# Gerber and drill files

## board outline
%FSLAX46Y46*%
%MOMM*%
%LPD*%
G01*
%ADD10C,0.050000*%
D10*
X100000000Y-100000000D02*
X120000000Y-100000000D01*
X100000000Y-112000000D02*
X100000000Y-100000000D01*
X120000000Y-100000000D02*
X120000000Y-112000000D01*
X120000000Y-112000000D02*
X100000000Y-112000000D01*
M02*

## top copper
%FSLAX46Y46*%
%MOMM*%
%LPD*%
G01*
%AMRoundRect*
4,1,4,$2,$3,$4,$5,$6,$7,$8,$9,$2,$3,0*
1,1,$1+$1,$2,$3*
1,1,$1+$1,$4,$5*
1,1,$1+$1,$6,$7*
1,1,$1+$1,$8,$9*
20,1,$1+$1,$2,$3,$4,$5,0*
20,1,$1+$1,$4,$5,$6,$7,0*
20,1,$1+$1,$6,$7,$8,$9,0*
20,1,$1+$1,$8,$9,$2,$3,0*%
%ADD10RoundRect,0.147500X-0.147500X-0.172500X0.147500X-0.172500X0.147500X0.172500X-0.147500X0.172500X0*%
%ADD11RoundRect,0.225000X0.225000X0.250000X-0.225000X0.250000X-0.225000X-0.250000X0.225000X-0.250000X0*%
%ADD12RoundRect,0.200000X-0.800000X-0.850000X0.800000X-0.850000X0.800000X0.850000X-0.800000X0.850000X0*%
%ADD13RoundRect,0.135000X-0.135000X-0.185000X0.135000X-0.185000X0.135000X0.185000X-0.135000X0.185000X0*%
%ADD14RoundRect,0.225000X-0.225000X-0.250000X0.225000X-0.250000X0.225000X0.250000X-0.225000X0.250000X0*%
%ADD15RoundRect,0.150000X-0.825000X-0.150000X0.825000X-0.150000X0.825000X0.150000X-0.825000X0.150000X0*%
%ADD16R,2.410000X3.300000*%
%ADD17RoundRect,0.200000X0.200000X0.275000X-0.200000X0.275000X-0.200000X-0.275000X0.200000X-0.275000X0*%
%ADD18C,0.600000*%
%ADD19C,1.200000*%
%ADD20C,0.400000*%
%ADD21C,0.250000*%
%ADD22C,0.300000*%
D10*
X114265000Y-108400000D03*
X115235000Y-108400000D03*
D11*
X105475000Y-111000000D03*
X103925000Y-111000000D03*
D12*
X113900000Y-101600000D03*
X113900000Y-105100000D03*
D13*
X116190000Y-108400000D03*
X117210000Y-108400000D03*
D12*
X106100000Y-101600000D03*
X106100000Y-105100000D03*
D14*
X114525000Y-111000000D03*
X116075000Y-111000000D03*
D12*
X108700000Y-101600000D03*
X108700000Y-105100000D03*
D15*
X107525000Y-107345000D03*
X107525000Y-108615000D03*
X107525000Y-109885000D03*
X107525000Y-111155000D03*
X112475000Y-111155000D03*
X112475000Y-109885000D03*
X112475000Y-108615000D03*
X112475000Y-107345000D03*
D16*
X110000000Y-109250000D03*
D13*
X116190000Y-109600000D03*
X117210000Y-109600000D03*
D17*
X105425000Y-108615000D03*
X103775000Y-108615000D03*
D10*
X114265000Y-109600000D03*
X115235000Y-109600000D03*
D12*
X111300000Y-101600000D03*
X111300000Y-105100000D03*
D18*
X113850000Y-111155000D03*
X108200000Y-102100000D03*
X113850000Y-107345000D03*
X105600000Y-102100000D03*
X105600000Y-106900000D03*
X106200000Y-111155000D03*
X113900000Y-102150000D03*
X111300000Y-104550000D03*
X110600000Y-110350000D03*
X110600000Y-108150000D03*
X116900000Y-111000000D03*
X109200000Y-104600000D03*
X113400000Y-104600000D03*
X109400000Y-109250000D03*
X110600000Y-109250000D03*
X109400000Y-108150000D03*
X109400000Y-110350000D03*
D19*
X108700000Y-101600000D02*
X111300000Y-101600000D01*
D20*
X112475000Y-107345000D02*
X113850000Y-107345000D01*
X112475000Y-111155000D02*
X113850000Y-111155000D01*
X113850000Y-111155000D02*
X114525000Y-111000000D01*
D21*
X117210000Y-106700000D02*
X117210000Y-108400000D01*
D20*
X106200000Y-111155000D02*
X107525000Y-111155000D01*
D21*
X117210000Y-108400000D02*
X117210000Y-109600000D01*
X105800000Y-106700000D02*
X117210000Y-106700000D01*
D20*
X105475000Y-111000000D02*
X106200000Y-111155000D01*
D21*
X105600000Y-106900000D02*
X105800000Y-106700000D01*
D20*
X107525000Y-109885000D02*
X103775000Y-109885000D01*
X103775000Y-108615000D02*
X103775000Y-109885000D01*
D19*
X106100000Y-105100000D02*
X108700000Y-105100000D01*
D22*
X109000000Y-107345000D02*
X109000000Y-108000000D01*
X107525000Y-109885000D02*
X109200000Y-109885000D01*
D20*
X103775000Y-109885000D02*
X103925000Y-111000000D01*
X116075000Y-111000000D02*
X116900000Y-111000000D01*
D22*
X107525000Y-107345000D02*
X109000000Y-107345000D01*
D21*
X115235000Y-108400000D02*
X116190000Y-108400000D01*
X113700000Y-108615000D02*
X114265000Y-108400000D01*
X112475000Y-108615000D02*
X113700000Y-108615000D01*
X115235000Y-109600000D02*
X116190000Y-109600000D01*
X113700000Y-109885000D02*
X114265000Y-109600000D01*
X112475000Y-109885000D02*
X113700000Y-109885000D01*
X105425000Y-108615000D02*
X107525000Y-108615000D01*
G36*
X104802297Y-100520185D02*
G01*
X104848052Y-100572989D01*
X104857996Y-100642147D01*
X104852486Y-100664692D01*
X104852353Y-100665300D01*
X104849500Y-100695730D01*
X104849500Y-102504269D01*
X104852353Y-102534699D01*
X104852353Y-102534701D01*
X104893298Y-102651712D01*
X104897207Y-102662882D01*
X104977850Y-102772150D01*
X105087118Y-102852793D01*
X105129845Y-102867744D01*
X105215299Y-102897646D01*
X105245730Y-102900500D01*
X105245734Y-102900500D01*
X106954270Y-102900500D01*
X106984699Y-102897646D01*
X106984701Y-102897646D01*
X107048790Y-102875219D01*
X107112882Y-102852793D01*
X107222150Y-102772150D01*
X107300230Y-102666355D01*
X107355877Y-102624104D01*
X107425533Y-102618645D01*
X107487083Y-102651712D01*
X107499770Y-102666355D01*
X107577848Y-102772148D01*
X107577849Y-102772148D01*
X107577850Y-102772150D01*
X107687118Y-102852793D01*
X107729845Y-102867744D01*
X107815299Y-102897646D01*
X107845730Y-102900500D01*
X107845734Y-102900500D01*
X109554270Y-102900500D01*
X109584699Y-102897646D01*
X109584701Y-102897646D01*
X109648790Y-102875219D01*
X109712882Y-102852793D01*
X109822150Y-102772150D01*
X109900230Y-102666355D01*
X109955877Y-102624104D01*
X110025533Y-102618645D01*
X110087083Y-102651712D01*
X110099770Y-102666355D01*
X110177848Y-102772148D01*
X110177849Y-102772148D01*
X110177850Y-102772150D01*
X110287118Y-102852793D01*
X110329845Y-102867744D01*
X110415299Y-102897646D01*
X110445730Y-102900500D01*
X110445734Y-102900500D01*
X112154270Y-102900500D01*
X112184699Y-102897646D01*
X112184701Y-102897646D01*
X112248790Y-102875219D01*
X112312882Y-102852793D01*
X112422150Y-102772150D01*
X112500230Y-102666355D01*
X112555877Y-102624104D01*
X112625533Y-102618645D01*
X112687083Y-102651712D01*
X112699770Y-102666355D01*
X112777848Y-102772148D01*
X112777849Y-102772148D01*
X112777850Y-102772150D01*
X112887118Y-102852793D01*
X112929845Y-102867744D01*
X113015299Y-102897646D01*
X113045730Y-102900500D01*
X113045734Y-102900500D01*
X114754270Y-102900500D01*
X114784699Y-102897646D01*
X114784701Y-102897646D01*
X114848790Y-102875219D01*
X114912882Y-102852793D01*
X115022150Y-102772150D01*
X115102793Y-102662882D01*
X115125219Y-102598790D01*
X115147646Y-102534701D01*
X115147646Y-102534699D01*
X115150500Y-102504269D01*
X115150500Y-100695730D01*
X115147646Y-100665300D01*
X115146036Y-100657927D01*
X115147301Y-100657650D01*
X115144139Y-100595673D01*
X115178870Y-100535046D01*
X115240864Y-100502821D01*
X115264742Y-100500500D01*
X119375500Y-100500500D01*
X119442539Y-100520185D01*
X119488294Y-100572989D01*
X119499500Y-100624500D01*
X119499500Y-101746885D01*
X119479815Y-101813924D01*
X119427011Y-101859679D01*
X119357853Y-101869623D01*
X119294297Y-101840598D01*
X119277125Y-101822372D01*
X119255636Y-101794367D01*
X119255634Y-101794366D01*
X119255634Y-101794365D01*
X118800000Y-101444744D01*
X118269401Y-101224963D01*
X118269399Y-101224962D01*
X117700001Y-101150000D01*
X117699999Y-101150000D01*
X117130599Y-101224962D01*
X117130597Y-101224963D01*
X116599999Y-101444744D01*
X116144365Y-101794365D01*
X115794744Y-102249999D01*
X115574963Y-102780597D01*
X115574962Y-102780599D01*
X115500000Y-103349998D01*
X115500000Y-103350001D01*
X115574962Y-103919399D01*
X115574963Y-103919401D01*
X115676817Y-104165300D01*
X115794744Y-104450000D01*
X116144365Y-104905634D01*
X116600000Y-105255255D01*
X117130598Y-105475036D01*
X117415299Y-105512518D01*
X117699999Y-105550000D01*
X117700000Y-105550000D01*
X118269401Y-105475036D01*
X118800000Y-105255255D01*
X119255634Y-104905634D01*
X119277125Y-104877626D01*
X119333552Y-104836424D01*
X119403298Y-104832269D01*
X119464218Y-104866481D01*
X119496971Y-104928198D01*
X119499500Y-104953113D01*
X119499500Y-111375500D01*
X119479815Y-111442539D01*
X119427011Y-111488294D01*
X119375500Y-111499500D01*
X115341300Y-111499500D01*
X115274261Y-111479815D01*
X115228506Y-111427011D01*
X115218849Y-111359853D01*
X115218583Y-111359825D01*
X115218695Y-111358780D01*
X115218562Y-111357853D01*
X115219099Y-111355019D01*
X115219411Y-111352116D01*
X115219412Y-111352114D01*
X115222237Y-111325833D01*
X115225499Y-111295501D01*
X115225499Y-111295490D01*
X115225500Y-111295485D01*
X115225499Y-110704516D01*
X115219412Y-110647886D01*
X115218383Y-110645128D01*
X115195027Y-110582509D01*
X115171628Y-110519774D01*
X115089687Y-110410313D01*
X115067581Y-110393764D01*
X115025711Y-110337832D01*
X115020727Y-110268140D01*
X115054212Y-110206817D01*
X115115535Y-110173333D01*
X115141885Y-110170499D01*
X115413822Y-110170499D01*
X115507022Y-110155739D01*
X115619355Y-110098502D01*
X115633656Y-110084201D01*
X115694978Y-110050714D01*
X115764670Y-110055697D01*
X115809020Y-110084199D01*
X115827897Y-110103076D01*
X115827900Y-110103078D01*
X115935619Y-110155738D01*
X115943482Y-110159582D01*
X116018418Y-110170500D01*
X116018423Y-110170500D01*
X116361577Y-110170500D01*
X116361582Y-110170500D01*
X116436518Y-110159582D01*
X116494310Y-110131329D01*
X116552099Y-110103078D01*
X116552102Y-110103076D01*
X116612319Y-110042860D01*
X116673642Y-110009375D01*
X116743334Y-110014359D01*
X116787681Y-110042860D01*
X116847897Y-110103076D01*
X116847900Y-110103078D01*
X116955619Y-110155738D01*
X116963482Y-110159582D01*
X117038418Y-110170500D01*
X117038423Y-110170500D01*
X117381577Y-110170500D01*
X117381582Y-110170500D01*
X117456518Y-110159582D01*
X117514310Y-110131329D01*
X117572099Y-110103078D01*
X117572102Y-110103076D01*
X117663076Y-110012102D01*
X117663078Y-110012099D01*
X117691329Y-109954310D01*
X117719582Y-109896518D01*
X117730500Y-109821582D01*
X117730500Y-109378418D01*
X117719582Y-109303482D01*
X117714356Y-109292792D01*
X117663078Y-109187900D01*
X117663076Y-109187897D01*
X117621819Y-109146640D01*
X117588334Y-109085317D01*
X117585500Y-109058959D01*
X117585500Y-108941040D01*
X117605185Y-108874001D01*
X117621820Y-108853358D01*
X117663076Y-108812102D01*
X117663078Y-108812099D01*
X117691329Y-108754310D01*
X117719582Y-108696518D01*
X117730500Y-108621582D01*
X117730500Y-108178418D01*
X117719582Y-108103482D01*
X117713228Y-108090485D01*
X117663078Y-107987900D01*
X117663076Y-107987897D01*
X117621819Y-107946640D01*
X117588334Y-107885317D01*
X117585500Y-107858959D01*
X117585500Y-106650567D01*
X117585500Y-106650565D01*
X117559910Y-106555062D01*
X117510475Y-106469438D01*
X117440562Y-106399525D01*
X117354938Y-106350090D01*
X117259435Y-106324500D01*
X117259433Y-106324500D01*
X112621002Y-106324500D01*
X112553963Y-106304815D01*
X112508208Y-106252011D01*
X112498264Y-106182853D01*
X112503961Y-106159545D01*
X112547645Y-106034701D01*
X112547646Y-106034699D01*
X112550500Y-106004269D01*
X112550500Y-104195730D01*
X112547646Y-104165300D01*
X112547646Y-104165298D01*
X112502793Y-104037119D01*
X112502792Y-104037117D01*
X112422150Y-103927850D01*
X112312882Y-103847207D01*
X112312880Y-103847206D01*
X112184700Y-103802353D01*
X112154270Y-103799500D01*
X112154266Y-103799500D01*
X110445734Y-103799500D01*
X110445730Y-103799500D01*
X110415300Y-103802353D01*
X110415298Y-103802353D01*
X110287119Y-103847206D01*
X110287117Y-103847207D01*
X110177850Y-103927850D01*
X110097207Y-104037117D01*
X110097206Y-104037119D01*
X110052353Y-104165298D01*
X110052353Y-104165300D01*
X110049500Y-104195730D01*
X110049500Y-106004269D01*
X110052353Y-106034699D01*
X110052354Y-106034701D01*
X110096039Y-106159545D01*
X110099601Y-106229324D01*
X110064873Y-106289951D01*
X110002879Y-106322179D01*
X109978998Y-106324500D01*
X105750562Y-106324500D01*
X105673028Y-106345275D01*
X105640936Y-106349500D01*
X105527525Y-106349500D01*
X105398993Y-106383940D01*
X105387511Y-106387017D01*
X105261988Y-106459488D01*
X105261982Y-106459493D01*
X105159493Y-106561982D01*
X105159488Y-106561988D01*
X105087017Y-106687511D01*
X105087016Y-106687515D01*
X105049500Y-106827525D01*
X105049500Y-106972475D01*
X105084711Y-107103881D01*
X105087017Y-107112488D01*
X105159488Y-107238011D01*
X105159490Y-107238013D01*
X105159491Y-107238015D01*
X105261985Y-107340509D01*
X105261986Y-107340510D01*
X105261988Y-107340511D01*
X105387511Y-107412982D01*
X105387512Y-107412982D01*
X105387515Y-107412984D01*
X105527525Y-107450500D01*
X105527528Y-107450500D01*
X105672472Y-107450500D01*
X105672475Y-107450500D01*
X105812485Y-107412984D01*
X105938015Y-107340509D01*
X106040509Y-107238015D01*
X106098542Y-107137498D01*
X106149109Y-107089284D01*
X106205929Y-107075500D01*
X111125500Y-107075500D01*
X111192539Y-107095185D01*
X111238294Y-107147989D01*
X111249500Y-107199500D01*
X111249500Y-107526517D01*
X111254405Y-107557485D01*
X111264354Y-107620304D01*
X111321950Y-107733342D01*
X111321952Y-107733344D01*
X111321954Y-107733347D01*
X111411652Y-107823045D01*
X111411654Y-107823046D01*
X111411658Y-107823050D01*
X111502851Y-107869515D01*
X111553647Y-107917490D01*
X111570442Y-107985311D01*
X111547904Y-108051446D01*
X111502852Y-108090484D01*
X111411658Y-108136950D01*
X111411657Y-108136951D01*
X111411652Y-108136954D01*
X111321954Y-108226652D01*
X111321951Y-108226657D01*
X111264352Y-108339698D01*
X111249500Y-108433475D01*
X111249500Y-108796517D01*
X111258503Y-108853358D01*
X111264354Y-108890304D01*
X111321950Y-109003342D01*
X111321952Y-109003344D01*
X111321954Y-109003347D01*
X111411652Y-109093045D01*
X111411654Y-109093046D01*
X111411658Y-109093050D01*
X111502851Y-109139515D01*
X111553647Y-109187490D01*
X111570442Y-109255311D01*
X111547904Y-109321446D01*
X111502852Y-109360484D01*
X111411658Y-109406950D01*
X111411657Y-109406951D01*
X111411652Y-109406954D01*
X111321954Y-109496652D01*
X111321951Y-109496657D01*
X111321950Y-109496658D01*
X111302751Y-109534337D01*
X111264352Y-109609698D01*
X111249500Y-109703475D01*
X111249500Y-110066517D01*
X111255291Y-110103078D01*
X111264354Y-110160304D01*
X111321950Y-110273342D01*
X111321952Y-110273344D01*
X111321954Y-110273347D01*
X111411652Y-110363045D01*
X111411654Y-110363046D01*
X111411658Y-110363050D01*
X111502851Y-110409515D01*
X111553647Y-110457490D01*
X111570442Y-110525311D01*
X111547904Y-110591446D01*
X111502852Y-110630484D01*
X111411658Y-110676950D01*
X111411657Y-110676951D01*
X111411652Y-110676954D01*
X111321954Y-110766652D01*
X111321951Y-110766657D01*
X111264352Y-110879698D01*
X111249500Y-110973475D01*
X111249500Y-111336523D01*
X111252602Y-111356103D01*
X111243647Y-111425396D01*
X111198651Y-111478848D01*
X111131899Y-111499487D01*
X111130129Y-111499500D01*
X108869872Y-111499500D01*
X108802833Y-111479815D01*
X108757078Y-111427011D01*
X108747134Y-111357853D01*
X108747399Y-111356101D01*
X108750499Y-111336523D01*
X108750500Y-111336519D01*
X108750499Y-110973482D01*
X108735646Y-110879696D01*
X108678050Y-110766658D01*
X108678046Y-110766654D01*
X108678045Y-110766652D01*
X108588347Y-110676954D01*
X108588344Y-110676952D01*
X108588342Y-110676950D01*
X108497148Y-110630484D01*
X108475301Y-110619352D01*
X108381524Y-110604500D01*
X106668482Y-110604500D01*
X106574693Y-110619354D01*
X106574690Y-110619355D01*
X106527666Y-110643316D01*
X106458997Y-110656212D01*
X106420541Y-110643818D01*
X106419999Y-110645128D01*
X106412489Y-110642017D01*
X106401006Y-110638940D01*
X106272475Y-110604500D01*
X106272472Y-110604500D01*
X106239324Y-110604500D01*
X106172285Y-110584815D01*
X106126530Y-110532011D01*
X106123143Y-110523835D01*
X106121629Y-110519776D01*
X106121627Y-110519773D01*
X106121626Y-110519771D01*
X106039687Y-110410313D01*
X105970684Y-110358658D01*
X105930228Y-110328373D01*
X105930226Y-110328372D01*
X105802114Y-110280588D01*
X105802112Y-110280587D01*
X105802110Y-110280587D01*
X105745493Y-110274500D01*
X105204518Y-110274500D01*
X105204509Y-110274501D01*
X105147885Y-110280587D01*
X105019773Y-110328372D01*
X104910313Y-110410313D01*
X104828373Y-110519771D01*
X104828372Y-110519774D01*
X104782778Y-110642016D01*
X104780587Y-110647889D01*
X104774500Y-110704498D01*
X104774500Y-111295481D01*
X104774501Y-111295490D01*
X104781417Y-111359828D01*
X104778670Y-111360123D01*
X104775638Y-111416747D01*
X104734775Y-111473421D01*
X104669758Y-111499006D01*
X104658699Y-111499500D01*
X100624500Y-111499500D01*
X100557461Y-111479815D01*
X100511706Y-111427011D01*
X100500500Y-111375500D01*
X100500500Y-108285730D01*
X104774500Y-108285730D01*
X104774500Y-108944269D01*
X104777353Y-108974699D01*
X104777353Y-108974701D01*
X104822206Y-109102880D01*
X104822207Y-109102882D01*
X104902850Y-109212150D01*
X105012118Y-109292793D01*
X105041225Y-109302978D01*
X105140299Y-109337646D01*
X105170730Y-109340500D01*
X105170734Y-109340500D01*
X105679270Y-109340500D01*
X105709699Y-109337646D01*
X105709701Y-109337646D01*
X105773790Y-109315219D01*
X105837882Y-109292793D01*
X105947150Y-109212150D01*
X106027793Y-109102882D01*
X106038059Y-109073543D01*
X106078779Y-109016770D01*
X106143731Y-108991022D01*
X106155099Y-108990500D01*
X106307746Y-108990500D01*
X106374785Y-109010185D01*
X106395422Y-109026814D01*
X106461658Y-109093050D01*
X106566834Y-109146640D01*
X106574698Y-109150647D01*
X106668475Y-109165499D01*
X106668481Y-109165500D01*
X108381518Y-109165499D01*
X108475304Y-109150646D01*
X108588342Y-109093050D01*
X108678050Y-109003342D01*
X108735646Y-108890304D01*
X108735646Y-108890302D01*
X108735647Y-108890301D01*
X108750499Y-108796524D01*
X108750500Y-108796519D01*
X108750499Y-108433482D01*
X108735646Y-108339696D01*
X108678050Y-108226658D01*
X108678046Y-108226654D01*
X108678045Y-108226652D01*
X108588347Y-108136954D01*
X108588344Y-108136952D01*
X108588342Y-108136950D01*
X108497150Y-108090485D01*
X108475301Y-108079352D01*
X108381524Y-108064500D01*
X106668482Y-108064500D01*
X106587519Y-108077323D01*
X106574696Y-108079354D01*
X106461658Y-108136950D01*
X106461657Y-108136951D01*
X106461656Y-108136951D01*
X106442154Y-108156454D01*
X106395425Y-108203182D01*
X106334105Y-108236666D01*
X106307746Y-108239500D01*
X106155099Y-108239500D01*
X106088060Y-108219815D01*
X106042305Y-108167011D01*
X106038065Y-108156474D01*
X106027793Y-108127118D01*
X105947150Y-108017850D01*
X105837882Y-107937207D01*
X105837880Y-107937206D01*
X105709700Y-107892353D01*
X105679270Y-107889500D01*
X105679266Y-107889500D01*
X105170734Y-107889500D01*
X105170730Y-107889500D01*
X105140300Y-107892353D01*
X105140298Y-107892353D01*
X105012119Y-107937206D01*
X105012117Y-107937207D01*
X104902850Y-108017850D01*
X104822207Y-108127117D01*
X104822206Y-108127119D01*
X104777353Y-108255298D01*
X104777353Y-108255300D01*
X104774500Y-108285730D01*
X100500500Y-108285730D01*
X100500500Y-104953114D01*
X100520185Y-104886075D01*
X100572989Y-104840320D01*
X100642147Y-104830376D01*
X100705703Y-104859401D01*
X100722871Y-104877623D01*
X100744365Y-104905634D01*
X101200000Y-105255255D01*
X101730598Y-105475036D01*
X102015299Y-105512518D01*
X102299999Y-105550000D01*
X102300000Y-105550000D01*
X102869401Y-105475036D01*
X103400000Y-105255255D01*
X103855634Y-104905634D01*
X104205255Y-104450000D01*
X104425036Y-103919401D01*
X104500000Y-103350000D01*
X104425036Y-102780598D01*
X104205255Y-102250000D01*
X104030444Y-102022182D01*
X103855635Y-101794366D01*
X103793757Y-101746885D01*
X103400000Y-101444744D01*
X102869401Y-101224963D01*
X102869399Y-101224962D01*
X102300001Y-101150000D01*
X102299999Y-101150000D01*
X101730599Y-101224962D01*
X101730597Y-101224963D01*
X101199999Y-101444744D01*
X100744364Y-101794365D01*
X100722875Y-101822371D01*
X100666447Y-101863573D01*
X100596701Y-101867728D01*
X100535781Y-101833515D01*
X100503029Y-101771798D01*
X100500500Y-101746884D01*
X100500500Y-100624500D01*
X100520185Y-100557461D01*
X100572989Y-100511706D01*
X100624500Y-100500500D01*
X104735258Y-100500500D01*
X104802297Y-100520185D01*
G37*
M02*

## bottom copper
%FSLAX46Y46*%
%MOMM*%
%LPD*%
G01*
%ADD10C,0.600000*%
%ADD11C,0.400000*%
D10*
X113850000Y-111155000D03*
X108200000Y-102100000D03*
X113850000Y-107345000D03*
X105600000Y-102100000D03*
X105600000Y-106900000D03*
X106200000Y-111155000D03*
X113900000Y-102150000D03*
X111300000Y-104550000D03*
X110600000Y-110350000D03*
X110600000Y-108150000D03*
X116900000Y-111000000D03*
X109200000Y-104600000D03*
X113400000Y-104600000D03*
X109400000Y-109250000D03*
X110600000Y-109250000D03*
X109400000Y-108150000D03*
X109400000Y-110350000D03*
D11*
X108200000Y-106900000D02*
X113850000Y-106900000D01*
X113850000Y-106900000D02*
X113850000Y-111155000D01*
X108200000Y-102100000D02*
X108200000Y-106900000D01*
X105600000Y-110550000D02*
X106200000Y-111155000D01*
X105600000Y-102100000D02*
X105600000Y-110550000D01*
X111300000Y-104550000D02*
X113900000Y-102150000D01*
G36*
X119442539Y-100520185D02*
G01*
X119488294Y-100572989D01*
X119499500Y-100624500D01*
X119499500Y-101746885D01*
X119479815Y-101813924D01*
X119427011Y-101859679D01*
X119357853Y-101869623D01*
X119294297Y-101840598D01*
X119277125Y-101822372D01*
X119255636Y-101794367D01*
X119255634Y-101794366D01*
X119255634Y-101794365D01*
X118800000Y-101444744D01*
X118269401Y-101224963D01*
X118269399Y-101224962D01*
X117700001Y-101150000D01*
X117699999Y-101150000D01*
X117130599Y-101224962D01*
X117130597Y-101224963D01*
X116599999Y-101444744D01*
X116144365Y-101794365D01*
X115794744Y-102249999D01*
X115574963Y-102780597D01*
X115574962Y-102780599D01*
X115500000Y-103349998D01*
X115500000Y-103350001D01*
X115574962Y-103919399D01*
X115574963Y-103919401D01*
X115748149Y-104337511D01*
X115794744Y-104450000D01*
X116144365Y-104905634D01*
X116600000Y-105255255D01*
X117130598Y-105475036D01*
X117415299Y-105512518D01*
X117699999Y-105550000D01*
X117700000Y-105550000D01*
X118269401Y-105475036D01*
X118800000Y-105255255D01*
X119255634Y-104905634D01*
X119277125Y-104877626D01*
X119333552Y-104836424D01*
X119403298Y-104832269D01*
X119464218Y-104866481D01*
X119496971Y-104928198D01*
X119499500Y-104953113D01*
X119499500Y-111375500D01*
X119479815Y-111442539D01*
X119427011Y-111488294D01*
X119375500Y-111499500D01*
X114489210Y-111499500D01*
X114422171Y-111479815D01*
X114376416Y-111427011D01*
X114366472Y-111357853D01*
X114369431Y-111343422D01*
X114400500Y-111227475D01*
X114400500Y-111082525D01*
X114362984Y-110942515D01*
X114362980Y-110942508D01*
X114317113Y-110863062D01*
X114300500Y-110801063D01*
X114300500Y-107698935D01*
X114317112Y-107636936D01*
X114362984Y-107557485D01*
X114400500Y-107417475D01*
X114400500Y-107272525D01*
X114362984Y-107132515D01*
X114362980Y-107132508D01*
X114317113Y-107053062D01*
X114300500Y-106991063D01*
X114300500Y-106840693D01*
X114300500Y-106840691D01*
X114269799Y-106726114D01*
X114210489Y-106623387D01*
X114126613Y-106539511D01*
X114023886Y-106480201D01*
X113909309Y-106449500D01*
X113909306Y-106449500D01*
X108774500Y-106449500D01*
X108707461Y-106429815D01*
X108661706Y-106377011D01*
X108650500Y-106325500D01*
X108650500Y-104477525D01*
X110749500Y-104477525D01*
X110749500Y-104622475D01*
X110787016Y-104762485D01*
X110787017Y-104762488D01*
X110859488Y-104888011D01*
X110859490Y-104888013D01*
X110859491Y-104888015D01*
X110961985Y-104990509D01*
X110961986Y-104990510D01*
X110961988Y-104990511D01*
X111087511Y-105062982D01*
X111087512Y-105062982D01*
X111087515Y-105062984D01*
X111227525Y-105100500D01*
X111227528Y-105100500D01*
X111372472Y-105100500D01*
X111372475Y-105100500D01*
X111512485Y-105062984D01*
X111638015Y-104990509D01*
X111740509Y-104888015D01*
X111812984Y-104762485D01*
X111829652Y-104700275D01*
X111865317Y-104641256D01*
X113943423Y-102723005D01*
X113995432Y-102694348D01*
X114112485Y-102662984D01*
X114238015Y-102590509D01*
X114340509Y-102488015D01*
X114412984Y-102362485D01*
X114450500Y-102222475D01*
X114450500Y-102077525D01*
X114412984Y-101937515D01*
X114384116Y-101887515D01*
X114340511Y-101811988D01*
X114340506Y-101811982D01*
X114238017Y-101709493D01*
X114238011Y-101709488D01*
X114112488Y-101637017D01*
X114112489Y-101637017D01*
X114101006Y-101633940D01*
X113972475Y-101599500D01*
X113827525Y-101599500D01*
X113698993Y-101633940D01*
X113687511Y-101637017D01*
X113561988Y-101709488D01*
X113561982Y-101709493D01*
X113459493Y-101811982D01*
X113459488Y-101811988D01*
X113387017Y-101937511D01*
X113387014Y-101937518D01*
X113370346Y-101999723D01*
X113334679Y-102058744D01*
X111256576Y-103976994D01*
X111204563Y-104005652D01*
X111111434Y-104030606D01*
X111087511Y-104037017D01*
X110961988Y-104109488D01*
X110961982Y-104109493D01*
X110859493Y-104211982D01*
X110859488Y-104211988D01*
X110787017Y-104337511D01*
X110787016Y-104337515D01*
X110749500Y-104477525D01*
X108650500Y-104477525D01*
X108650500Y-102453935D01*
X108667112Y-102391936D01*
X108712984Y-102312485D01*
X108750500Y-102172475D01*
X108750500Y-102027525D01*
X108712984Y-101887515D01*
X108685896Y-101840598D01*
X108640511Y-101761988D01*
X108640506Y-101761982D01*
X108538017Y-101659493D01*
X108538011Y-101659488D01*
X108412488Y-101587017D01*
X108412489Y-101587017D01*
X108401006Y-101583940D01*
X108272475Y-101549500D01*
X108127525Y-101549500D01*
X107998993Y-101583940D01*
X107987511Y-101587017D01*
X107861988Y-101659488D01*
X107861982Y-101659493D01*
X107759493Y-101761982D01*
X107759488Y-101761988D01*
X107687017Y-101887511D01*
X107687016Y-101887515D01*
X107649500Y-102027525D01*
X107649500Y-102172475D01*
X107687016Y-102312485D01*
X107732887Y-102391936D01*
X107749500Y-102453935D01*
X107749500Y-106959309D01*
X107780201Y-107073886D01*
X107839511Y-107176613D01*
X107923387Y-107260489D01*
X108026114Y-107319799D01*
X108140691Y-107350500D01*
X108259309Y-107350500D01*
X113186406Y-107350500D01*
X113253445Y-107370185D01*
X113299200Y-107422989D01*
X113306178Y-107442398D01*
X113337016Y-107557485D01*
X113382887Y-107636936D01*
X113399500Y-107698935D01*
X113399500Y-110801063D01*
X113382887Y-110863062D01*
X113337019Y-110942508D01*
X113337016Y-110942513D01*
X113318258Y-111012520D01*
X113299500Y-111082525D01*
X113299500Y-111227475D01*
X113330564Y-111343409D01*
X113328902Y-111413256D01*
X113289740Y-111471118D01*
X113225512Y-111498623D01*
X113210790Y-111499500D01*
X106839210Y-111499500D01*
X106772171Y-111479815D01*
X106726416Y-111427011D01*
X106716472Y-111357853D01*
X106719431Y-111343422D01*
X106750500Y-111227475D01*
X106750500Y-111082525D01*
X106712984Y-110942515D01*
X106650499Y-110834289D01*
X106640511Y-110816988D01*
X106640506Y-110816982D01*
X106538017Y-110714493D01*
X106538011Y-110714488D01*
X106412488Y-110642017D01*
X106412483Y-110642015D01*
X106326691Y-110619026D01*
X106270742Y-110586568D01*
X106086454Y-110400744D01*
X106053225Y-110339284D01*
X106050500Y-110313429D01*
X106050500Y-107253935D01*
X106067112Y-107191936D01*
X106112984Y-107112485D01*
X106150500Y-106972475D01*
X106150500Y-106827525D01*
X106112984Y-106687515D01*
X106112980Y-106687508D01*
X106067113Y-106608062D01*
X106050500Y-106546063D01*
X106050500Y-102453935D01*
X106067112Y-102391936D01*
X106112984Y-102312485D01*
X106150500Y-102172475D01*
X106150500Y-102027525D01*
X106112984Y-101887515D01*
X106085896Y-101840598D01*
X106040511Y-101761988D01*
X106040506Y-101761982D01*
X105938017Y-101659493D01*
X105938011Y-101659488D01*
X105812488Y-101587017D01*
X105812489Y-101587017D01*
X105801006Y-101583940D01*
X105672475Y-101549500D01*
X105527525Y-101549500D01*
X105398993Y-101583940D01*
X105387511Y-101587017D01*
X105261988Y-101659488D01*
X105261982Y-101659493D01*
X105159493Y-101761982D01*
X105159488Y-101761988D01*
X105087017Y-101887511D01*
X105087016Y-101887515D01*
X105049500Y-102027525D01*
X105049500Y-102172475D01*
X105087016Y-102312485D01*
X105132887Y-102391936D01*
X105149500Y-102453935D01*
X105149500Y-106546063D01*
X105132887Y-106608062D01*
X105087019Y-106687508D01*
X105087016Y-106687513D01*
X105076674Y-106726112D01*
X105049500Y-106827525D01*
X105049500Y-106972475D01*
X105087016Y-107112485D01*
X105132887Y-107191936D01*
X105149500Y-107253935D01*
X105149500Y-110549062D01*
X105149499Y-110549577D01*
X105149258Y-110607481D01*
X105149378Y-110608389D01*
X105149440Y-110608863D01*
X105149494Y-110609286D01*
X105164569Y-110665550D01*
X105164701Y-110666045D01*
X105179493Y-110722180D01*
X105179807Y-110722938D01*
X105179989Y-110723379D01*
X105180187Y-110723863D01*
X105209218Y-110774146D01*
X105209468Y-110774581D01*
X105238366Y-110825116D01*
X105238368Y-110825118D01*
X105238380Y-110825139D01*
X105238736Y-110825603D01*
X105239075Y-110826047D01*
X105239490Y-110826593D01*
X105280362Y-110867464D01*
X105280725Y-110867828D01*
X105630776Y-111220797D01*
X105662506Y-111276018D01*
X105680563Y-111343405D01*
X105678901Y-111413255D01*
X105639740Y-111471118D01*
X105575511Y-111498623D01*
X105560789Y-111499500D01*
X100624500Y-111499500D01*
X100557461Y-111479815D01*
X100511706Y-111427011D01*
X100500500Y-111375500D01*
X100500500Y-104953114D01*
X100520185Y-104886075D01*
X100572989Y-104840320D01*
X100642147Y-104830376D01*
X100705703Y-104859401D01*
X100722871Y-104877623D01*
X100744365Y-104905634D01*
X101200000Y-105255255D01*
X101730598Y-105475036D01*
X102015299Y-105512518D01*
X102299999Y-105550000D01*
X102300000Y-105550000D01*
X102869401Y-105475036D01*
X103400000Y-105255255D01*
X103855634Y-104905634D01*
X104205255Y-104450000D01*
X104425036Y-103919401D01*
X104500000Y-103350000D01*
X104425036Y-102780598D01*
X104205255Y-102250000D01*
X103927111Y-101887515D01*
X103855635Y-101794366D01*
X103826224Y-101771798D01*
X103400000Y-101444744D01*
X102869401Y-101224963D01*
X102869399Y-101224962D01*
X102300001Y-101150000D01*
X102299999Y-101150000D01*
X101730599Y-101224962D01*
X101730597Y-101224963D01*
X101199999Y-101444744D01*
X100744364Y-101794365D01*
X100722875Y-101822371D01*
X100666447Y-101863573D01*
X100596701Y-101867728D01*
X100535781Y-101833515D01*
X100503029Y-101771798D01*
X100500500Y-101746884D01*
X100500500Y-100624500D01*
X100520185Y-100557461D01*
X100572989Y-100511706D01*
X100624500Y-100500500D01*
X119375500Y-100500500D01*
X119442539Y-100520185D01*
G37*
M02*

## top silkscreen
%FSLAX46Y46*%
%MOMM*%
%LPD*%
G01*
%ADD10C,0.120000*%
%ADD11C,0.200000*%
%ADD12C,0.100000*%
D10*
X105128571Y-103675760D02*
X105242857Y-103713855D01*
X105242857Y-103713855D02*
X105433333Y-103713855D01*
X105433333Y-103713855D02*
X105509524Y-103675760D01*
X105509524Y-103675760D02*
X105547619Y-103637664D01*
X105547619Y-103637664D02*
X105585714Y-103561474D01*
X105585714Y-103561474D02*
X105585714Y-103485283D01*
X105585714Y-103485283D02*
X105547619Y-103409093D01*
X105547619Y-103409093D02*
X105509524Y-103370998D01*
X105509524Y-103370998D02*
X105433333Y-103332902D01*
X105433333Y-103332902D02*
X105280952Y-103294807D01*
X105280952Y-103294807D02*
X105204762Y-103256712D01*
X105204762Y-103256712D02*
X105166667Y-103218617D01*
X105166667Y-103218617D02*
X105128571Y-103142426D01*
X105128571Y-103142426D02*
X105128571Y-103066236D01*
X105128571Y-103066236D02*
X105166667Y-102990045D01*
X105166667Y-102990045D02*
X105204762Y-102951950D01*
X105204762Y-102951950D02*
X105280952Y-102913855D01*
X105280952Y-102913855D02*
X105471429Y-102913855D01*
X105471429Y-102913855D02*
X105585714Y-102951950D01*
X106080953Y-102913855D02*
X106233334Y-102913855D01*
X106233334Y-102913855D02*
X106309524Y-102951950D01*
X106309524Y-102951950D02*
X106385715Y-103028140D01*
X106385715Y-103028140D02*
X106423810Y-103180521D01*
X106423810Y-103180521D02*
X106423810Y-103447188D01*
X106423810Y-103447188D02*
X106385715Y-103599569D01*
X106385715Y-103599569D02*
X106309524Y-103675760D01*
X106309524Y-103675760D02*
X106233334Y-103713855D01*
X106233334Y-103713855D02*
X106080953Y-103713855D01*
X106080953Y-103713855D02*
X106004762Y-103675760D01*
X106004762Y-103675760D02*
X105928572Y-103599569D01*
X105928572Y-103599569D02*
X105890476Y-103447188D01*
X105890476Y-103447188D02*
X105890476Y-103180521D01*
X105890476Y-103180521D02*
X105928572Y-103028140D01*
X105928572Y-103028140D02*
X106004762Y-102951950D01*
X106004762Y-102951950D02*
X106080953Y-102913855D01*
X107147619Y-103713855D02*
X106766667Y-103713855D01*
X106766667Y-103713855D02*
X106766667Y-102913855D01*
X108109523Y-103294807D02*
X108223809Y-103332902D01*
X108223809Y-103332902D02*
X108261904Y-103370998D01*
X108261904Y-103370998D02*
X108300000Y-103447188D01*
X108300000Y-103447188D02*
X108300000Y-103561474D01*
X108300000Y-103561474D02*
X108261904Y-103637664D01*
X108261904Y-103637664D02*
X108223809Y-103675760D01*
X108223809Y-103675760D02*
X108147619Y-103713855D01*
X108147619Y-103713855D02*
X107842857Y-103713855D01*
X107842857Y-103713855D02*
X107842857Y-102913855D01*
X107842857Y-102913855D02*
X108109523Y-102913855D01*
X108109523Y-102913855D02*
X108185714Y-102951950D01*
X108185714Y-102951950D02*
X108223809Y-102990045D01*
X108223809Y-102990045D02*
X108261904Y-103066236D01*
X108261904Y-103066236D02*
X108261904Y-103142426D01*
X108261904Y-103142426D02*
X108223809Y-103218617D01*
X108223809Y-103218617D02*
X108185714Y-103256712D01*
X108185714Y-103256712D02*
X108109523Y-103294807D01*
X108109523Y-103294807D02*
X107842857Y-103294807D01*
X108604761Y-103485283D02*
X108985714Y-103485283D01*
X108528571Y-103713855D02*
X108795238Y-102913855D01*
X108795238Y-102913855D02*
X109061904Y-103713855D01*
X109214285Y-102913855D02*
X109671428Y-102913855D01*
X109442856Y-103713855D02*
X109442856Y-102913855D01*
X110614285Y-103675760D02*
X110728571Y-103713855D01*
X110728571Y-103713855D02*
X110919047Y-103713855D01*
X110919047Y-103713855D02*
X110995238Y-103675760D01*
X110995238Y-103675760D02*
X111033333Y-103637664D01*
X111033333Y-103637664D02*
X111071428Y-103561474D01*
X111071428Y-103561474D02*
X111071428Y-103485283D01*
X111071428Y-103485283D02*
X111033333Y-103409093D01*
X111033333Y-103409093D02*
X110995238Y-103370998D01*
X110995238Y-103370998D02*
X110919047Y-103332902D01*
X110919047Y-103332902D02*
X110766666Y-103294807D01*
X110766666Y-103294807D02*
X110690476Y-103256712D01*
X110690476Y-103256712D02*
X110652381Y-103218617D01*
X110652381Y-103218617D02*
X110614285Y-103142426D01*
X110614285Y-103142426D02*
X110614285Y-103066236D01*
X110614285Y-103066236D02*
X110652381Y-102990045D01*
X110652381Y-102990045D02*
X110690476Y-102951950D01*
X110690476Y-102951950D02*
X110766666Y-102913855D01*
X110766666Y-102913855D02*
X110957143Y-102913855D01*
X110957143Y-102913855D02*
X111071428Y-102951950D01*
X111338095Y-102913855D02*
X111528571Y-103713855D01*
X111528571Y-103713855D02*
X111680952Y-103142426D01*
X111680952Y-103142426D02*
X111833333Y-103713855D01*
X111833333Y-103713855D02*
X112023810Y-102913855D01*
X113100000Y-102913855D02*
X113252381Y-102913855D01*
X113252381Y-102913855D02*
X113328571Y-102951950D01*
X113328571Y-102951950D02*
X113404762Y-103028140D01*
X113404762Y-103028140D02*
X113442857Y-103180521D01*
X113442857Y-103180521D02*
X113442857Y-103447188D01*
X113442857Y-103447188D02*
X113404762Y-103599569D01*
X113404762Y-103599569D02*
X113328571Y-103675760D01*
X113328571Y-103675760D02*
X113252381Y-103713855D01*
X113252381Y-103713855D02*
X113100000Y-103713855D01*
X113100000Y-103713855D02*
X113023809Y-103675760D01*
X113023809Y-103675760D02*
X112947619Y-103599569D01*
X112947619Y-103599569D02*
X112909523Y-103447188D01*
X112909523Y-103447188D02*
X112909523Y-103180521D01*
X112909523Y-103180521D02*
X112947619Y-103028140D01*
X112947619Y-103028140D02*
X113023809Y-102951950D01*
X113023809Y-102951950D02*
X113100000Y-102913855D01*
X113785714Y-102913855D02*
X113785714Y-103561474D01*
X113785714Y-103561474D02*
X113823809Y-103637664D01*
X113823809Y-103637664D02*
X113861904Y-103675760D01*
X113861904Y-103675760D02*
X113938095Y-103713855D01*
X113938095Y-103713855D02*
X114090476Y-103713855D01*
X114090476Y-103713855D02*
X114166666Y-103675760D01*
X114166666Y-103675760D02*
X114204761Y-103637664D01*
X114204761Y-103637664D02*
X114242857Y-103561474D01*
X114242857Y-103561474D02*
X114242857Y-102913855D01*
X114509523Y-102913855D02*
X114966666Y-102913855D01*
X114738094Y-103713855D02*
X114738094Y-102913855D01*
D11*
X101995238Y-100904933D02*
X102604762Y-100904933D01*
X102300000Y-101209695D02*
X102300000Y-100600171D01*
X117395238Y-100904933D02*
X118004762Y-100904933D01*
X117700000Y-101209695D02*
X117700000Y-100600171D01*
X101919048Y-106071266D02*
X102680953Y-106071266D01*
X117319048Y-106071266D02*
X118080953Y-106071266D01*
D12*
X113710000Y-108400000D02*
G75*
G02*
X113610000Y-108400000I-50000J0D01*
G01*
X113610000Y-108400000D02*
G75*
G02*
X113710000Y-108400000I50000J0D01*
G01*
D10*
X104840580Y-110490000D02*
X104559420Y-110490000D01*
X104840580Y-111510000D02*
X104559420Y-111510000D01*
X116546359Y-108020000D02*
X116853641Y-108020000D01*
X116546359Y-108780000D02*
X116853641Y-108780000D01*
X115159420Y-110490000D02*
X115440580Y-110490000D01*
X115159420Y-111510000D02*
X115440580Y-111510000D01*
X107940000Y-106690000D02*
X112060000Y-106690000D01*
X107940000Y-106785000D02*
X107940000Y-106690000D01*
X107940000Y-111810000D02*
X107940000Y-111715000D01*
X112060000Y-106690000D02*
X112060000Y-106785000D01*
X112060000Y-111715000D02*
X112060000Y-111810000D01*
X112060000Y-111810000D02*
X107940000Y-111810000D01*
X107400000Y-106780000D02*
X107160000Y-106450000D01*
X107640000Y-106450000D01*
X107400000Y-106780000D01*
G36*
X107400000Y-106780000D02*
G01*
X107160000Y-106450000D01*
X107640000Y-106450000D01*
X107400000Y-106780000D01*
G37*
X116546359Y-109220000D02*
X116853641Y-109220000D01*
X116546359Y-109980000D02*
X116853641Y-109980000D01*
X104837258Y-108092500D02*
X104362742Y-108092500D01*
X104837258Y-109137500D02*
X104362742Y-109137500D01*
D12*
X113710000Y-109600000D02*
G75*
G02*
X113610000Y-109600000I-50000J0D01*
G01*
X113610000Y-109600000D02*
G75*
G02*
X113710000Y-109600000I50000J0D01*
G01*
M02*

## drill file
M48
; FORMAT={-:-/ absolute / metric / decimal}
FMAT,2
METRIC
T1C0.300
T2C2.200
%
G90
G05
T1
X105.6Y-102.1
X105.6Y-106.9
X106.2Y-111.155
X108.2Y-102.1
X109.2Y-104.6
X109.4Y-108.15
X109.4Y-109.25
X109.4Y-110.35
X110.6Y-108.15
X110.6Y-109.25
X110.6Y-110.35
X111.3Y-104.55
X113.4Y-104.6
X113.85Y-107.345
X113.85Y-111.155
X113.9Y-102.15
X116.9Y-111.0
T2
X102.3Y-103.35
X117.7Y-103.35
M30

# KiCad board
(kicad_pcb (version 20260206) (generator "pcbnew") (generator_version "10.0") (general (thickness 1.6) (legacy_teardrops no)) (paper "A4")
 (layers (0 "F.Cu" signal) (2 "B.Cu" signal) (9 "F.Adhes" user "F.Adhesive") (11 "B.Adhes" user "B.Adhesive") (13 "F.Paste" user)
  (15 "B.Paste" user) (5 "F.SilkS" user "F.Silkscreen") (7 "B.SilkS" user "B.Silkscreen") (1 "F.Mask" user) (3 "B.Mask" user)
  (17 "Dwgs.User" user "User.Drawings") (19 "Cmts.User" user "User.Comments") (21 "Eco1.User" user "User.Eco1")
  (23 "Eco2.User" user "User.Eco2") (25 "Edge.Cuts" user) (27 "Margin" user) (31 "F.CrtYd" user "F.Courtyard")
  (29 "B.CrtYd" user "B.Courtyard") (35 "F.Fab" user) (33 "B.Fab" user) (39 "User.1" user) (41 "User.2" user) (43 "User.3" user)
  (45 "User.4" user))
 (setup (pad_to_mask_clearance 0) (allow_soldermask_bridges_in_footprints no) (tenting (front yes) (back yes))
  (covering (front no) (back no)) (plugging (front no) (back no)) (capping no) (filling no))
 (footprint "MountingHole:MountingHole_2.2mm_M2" (layer "F.Cu") (at 102.3 103.35)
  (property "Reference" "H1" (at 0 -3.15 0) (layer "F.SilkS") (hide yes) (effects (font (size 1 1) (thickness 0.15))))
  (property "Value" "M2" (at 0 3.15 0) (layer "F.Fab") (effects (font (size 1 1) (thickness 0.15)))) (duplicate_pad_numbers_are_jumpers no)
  (pad "" np_thru_hole circle (at 0 0) (size 2.2 2.2) (drill 2.2) (layers "*.Cu" "*.Mask")))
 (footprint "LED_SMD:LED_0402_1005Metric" (layer "F.Cu") (at 114.75 108.4)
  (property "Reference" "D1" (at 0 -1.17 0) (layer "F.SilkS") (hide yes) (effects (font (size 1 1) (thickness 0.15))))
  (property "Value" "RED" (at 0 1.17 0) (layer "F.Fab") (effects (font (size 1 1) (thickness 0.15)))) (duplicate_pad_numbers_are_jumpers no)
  (fp_circle (center -1.09 0) (end -1.04 0) (stroke (width 0.1) (type solid)) (fill no) (layer "F.SilkS"))
  (pad "1" smd roundrect (at -0.485 0) (size 0.59 0.64) (layers "F.Cu" "F.Mask" "F.Paste") (roundrect_rratio 0.25) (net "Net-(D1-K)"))
  (pad "2" smd roundrect (at 0.485 0) (size 0.59 0.64) (layers "F.Cu" "F.Mask" "F.Paste") (roundrect_rratio 0.25) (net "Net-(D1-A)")))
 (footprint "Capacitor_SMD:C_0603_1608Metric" (layer "F.Cu") (at 104.7 111 180)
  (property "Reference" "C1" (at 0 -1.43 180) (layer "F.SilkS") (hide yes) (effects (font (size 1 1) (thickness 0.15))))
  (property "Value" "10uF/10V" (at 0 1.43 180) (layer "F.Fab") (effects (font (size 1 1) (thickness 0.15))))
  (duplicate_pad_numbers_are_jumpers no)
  (fp_line (start -0.14058 0.51) (end 0.14058 0.51) (stroke (width 0.12) (type solid)) (layer "F.SilkS"))
  (fp_line (start -0.14058 -0.51) (end 0.14058 -0.51) (stroke (width 0.12) (type solid)) (layer "F.SilkS"))
  (pad "1" smd roundrect (at -0.775 0 180) (size 0.9 0.95) (layers "F.Cu" "F.Mask" "F.Paste") (roundrect_rratio 0.25) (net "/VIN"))
  (pad "2" smd roundrect (at 0.775 0 180) (size 0.9 0.95) (layers "F.Cu" "F.Mask" "F.Paste") (roundrect_rratio 0.25) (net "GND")))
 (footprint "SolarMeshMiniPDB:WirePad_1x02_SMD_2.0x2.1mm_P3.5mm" (layer "F.Cu") (at 113.9 103.35)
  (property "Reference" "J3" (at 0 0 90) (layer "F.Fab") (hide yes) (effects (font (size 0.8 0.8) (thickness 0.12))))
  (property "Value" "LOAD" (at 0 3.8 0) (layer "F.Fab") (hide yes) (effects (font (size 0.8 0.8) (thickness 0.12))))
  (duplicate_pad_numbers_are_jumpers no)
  (pad "1" smd roundrect (at 0 -1.75) (size 2 2.1) (layers "F.Cu" "F.Mask") (roundrect_rratio 0.1) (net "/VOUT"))
  (pad "2" smd roundrect (at 0 1.75) (size 2 2.1) (layers "F.Cu" "F.Mask") (roundrect_rratio 0.1) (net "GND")))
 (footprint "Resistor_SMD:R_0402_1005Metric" (layer "F.Cu") (at 116.7 108.4)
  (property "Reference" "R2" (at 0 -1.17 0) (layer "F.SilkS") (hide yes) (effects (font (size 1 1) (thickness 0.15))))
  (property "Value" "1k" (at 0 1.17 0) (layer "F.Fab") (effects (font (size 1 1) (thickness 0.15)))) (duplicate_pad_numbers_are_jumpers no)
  (fp_line (start -0.153641 -0.38) (end 0.153641 -0.38) (stroke (width 0.12) (type solid)) (layer "F.SilkS"))
  (fp_line (start -0.153641 0.38) (end 0.153641 0.38) (stroke (width 0.12) (type solid)) (layer "F.SilkS"))
  (pad "1" smd roundrect (at -0.51 0) (size 0.54 0.64) (layers "F.Cu" "F.Mask" "F.Paste") (roundrect_rratio 0.25) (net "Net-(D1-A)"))
  (pad "2" smd roundrect (at 0.51 0) (size 0.54 0.64) (layers "F.Cu" "F.Mask" "F.Paste") (roundrect_rratio 0.25) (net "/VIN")))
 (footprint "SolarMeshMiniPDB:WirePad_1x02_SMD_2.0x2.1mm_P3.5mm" (layer "F.Cu") (at 106.1 103.35)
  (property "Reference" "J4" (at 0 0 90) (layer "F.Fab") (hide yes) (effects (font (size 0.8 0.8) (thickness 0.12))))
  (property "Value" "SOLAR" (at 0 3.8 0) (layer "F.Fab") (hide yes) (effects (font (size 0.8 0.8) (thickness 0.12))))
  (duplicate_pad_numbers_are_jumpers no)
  (pad "1" smd roundrect (at 0 -1.75) (size 2 2.1) (layers "F.Cu" "F.Mask") (roundrect_rratio 0.1) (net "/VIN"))
  (pad "2" smd roundrect (at 0 1.75) (size 2 2.1) (layers "F.Cu" "F.Mask") (roundrect_rratio 0.1) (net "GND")))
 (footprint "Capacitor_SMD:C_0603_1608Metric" (layer "F.Cu") (at 115.3 111)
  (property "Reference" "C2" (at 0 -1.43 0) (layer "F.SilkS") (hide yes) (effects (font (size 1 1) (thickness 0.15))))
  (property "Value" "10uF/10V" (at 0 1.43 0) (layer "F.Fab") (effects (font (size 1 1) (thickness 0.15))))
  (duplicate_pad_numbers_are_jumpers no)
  (fp_line (start -0.14058 -0.51) (end 0.14058 -0.51) (stroke (width 0.12) (type solid)) (layer "F.SilkS"))
  (fp_line (start -0.14058 0.51) (end 0.14058 0.51) (stroke (width 0.12) (type solid)) (layer "F.SilkS"))
  (pad "1" smd roundrect (at -0.775 0) (size 0.9 0.95) (layers "F.Cu" "F.Mask" "F.Paste") (roundrect_rratio 0.25) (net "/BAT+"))
  (pad "2" smd roundrect (at 0.775 0) (size 0.9 0.95) (layers "F.Cu" "F.Mask" "F.Paste") (roundrect_rratio 0.25) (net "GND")))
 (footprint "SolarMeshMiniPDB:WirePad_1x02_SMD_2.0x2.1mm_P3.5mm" (layer "F.Cu") (at 108.7 103.35)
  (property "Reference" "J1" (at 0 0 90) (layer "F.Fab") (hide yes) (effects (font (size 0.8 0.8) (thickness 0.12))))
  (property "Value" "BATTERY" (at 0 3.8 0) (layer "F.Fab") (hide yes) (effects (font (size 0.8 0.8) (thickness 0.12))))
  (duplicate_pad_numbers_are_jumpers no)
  (pad "1" smd roundrect (at 0 -1.75) (size 2 2.1) (layers "F.Cu" "F.Mask") (roundrect_rratio 0.1) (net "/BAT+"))
  (pad "2" smd roundrect (at 0 1.75) (size 2 2.1) (layers "F.Cu" "F.Mask") (roundrect_rratio 0.1) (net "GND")))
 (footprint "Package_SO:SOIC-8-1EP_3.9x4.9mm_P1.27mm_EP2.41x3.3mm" (layer "F.Cu") (at 110 109.25)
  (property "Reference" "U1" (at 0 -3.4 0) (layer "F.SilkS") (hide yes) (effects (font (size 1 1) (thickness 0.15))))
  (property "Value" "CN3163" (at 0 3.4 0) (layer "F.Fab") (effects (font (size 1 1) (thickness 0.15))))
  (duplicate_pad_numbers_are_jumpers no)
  (fp_line (start -2.06 -2.56) (end 2.06 -2.56) (stroke (width 0.12) (type solid)) (layer "F.SilkS"))
  (fp_line (start -2.06 -2.465) (end -2.06 -2.56) (stroke (width 0.12) (type solid)) (layer "F.SilkS"))
  (fp_line (start -2.06 2.56) (end -2.06 2.465) (stroke (width 0.12) (type solid)) (layer "F.SilkS"))
  (fp_line (start 2.06 -2.56) (end 2.06 -2.465) (stroke (width 0.12) (type solid)) (layer "F.SilkS"))
  (fp_line (start 2.06 2.465) (end 2.06 2.56) (stroke (width 0.12) (type solid)) (layer "F.SilkS"))
  (fp_line (start 2.06 2.56) (end -2.06 2.56) (stroke (width 0.12) (type solid)) (layer "F.SilkS"))
  (fp_poly (pts (xy -2.6 -2.47) (xy -2.84 -2.8) (xy -2.36 -2.8)) (stroke (width 0.12) (type solid)) (fill yes) (layer "F.SilkS"))
  (pad "" smd roundrect (at -0.6 -0.825) (size 0.97 1.33) (layers "F.Paste") (roundrect_rratio 0.25))
  (pad "" smd roundrect (at -0.6 0.825) (size 0.97 1.33) (layers "F.Paste") (roundrect_rratio 0.25))
  (pad "" smd roundrect (at 0.6 -0.825) (size 0.97 1.33) (layers "F.Paste") (roundrect_rratio 0.25))
  (pad "" smd roundrect (at 0.6 0.825) (size 0.97 1.33) (layers "F.Paste") (roundrect_rratio 0.25))
  (pad "1" smd roundrect (at -2.475 -1.905) (size 1.95 0.6) (layers "F.Cu" "F.Mask" "F.Paste") (roundrect_rratio 0.25) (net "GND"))
  (pad "2" smd roundrect (at -2.475 -0.635) (size 1.95 0.6) (layers "F.Cu" "F.Mask" "F.Paste") (roundrect_rratio 0.25) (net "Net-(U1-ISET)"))
  (pad "3" smd roundrect (at -2.475 0.635) (size 1.95 0.6) (layers "F.Cu" "F.Mask" "F.Paste") (roundrect_rratio 0.25) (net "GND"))
  (pad "4" smd roundrect (at -2.475 1.905) (size 1.95 0.6) (layers "F.Cu" "F.Mask" "F.Paste") (roundrect_rratio 0.25) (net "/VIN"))
  (pad "5" smd roundrect (at 2.475 1.905) (size 1.95 0.6) (layers "F.Cu" "F.Mask" "F.Paste") (roundrect_rratio 0.25) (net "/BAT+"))
  (pad "6" smd roundrect (at 2.475 0.635) (size 1.95 0.6) (layers "F.Cu" "F.Mask" "F.Paste") (roundrect_rratio 0.25) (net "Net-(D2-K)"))
  (pad "7" smd roundrect (at 2.475 -0.635) (size 1.95 0.6) (layers "F.Cu" "F.Mask" "F.Paste") (roundrect_rratio 0.25) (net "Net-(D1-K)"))
  (pad "8" smd roundrect (at 2.475 -1.905) (size 1.95 0.6) (layers "F.Cu" "F.Mask" "F.Paste") (roundrect_rratio 0.25) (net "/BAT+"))
  (pad "9" smd rect (at 0 0) (size 2.41 3.3) (layers "F.Cu" "F.Mask") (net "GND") (zone_connect 2)))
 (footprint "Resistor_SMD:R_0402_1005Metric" (layer "F.Cu") (at 116.7 109.6)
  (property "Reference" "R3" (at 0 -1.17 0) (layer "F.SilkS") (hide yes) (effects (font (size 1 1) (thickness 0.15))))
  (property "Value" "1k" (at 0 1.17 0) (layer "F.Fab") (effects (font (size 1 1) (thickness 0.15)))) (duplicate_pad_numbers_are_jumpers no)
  (fp_line (start -0.153641 -0.38) (end 0.153641 -0.38) (stroke (width 0.12) (type solid)) (layer "F.SilkS"))
  (fp_line (start -0.153641 0.38) (end 0.153641 0.38) (stroke (width 0.12) (type solid)) (layer "F.SilkS"))
  (pad "1" smd roundrect (at -0.51 0) (size 0.54 0.64) (layers "F.Cu" "F.Mask" "F.Paste") (roundrect_rratio 0.25) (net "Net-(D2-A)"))
  (pad "2" smd roundrect (at 0.51 0) (size 0.54 0.64) (layers "F.Cu" "F.Mask" "F.Paste") (roundrect_rratio 0.25) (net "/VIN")))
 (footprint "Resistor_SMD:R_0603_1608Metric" (layer "F.Cu") (at 104.6 108.615 180)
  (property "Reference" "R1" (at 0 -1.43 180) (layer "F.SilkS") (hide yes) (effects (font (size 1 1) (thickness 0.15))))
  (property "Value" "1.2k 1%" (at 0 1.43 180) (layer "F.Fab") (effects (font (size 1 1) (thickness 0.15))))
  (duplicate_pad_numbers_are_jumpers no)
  (fp_line (start -0.237258 0.5225) (end 0.237258 0.5225) (stroke (width 0.12) (type solid)) (layer "F.SilkS"))
  (fp_line (start -0.237258 -0.5225) (end 0.237258 -0.5225) (stroke (width 0.12) (type solid)) (layer "F.SilkS"))
  (pad "1" smd roundrect (at -0.825 0 180) (size 0.8 0.95) (layers "F.Cu" "F.Mask" "F.Paste") (roundrect_rratio 0.25) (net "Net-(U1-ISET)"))
  (pad "2" smd roundrect (at 0.825 0 180) (size 0.8 0.95) (layers "F.Cu" "F.Mask" "F.Paste") (roundrect_rratio 0.25) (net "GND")))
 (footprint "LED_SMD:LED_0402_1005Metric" (layer "F.Cu") (at 114.75 109.6)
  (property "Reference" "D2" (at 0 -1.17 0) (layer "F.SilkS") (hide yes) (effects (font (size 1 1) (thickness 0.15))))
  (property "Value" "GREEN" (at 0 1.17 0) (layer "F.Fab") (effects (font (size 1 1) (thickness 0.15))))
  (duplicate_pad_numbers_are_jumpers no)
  (fp_circle (center -1.09 0) (end -1.04 0) (stroke (width 0.1) (type solid)) (fill no) (layer "F.SilkS"))
  (pad "1" smd roundrect (at -0.485 0) (size 0.59 0.64) (layers "F.Cu" "F.Mask" "F.Paste") (roundrect_rratio 0.25) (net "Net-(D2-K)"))
  (pad "2" smd roundrect (at 0.485 0) (size 0.59 0.64) (layers "F.Cu" "F.Mask" "F.Paste") (roundrect_rratio 0.25) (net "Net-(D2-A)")))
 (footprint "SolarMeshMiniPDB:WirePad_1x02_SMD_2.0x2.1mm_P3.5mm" (layer "F.Cu") (at 111.3 103.35)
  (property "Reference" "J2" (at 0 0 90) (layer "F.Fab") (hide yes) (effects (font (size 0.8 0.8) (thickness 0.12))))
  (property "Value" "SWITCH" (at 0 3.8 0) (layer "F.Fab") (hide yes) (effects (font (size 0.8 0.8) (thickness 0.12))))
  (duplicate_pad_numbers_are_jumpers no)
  (pad "1" smd roundrect (at 0 -1.75) (size 2 2.1) (layers "F.Cu" "F.Mask") (roundrect_rratio 0.1) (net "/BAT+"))
  (pad "2" smd roundrect (at 0 1.75) (size 2 2.1) (layers "F.Cu" "F.Mask") (roundrect_rratio 0.1) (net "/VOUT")))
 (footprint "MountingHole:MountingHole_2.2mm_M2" (layer "F.Cu") (at 117.7 103.35)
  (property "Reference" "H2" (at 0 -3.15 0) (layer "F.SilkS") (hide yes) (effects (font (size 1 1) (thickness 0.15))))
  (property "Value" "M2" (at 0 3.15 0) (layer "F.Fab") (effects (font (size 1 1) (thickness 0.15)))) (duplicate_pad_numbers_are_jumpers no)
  (pad "" np_thru_hole circle (at 0 0) (size 2.2 2.2) (drill 2.2) (layers "*.Cu" "*.Mask")))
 (gr_line (start 100 100) (end 120 100) (stroke (width 0.05) (type default)) (layer "Edge.Cuts"))
 (gr_line (start 100 112) (end 100 100) (stroke (width 0.05) (type default)) (layer "Edge.Cuts"))
 (gr_line (start 120 100) (end 120 112) (stroke (width 0.05) (type default)) (layer "Edge.Cuts"))
 (gr_line (start 120 112) (end 100 112) (stroke (width 0.05) (type default)) (layer "Edge.Cuts"))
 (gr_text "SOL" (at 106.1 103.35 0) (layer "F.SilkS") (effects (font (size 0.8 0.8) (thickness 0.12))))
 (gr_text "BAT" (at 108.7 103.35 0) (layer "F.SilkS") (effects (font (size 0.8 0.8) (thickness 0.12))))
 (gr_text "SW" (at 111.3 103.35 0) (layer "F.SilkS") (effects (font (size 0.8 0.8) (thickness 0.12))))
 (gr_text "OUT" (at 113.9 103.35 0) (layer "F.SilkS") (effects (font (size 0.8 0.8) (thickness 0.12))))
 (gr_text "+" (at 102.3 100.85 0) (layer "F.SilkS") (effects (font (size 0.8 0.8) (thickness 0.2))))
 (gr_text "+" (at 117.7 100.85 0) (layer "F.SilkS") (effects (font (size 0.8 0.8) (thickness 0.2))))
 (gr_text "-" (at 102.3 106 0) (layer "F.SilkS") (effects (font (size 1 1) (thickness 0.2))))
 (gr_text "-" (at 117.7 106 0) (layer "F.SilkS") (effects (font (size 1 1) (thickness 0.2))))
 (segment (start 108.7 101.6) (end 111.3 101.6) (width 1.2) (layer "F.Cu") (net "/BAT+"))
 (segment (start 112.475 107.345) (end 113.85 107.345) (width 0.4) (layer "F.Cu") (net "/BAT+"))
 (segment (start 112.475 111.155) (end 113.85 111.155) (width 0.4) (layer "F.Cu") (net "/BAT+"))
 (segment (start 113.85 111.155) (end 114.525 111) (width 0.4) (layer "F.Cu") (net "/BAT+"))
 (via (at 113.85 111.155) (size 0.6) (drill 0.3) (layers "F.Cu" "B.Cu") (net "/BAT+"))
 (via (at 108.2 102.1) (size 0.6) (drill 0.3) (layers "F.Cu" "B.Cu") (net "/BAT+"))
 (via (at 113.85 107.345) (size 0.6) (drill 0.3) (layers "F.Cu" "B.Cu") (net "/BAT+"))
 (segment (start 108.2 106.9) (end 113.85 106.9) (width 0.4) (layer "B.Cu") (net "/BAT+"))
 (segment (start 113.85 106.9) (end 113.85 111.155) (width 0.4) (layer "B.Cu") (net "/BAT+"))
 (segment (start 108.2 102.1) (end 108.2 106.9) (width 0.4) (layer "B.Cu") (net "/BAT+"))
 (segment (start 117.21 106.7) (end 117.21 108.4) (width 0.25) (layer "F.Cu") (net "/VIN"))
 (segment (start 106.2 111.155) (end 107.525 111.155) (width 0.4) (layer "F.Cu") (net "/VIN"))
 (segment (start 117.21 108.4) (end 117.21 109.6) (width 0.25) (layer "F.Cu") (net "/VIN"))
 (segment (start 105.8 106.7) (end 117.21 106.7) (width 0.25) (layer "F.Cu") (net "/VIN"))
 (segment (start 105.475 111) (end 106.2 111.155) (width 0.4) (layer "F.Cu") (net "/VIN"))
 (segment (start 105.6 106.9) (end 105.8 106.7) (width 0.25) (layer "F.Cu") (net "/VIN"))
 (via (at 105.6 102.1) (size 0.6) (drill 0.3) (layers "F.Cu" "B.Cu") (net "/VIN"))
 (via (at 105.6 106.9) (size 0.6) (drill 0.3) (layers "F.Cu" "B.Cu") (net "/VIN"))
 (via (at 106.2 111.155) (size 0.6) (drill 0.3) (layers "F.Cu" "B.Cu") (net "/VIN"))
 (segment (start 105.6 110.55) (end 106.2 111.155) (width 0.4) (layer "B.Cu") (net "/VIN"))
 (segment (start 105.6 102.1) (end 105.6 110.55) (width 0.4) (layer "B.Cu") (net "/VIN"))
 (via (at 113.9 102.15) (size 0.6) (drill 0.3) (layers "F.Cu" "B.Cu") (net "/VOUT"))
 (via (at 111.3 104.55) (size 0.6) (drill 0.3) (layers "F.Cu" "B.Cu") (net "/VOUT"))
 (segment (start 111.3 104.55) (end 113.9 102.15) (width 0.4) (layer "B.Cu") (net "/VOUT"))
 (segment (start 107.525 109.885) (end 103.775 109.885) (width 0.4) (layer "F.Cu") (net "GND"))
 (segment (start 103.775 108.615) (end 103.775 109.885) (width 0.4) (layer "F.Cu") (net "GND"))
 (segment (start 106.1 105.1) (end 108.7 105.1) (width 1.2) (layer "F.Cu") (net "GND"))
 (segment (start 109 107.345) (end 109 108) (width 0.3) (layer "F.Cu") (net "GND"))
 (segment (start 107.525 109.885) (end 109.2 109.885) (width 0.3) (layer "F.Cu") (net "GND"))
 (segment (start 103.775 109.885) (end 103.925 111) (width 0.4) (layer "F.Cu") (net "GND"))
 (segment (start 116.075 111) (end 116.9 111) (width 0.4) (layer "F.Cu") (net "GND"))
 (segment (start 107.525 107.345) (end 109 107.345) (width 0.3) (layer "F.Cu") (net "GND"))
 (via (at 110.6 110.35) (size 0.6) (drill 0.3) (layers "F.Cu" "B.Cu") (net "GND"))
 (via (at 110.6 108.15) (size 0.6) (drill 0.3) (layers "F.Cu" "B.Cu") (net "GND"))
 (via (at 116.9 111) (size 0.6) (drill 0.3) (layers "F.Cu" "B.Cu") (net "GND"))
 (via (at 109.2 104.6) (size 0.6) (drill 0.3) (layers "F.Cu" "B.Cu") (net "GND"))
 (via (at 113.4 104.6) (size 0.6) (drill 0.3) (layers "F.Cu" "B.Cu") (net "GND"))
 (via (at 109.4 109.25) (size 0.6) (drill 0.3) (layers "F.Cu" "B.Cu") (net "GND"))
 (via (at 110.6 109.25) (size 0.6) (drill 0.3) (layers "F.Cu" "B.Cu") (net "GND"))
 (via (at 109.4 108.15) (size 0.6) (drill 0.3) (layers "F.Cu" "B.Cu") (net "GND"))
 (via (at 109.4 110.35) (size 0.6) (drill 0.3) (layers "F.Cu" "B.Cu") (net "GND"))
 (segment (start 115.235 108.4) (end 116.19 108.4) (width 0.25) (layer "F.Cu") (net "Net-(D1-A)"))
 (segment (start 113.7 108.615) (end 114.265 108.4) (width 0.25) (layer "F.Cu") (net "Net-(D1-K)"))
 (segment (start 112.475 108.615) (end 113.7 108.615) (width 0.25) (layer "F.Cu") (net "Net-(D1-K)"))
 (segment (start 115.235 109.6) (end 116.19 109.6) (width 0.25) (layer "F.Cu") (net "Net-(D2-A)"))
 (segment (start 113.7 109.885) (end 114.265 109.6) (width 0.25) (layer "F.Cu") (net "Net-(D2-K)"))
 (segment (start 112.475 109.885) (end 113.7 109.885) (width 0.25) (layer "F.Cu") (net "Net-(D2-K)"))
 (segment (start 105.425 108.615) (end 107.525 108.615) (width 0.25) (layer "F.Cu") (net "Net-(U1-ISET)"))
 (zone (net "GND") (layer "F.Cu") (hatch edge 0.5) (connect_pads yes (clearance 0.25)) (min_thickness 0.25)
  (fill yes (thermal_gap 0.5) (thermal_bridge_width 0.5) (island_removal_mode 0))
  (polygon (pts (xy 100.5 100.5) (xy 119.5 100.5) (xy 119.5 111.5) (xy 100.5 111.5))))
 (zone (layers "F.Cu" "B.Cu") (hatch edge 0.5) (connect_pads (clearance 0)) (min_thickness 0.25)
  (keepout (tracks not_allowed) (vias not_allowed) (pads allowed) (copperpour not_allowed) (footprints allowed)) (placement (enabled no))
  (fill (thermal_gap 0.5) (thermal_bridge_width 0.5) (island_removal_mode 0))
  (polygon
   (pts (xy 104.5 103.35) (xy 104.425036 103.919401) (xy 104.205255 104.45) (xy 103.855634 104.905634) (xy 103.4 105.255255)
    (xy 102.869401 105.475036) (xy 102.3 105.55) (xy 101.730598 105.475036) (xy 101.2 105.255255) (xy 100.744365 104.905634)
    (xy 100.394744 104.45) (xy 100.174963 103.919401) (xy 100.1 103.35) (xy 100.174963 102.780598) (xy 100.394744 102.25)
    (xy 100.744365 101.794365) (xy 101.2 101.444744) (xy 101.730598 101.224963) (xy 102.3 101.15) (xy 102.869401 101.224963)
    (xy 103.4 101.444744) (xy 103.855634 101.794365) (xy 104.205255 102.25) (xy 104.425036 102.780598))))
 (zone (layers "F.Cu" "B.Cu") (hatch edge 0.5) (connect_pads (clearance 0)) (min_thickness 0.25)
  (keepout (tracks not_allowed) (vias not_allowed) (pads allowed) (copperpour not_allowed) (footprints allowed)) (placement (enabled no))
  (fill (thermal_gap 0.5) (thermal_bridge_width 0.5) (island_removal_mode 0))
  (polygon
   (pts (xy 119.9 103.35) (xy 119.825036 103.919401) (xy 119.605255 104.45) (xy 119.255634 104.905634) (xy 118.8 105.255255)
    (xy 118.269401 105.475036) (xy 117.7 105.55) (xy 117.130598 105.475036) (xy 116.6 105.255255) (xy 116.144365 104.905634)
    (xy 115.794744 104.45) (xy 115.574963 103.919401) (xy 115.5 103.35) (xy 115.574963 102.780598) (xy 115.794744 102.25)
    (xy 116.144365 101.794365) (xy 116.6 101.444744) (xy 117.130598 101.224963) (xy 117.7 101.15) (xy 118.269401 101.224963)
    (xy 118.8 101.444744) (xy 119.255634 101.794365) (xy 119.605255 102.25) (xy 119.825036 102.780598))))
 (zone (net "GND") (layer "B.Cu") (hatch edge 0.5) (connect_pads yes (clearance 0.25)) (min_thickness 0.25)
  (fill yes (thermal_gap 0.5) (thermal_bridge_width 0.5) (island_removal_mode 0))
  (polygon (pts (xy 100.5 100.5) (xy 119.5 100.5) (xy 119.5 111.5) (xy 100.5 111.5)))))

